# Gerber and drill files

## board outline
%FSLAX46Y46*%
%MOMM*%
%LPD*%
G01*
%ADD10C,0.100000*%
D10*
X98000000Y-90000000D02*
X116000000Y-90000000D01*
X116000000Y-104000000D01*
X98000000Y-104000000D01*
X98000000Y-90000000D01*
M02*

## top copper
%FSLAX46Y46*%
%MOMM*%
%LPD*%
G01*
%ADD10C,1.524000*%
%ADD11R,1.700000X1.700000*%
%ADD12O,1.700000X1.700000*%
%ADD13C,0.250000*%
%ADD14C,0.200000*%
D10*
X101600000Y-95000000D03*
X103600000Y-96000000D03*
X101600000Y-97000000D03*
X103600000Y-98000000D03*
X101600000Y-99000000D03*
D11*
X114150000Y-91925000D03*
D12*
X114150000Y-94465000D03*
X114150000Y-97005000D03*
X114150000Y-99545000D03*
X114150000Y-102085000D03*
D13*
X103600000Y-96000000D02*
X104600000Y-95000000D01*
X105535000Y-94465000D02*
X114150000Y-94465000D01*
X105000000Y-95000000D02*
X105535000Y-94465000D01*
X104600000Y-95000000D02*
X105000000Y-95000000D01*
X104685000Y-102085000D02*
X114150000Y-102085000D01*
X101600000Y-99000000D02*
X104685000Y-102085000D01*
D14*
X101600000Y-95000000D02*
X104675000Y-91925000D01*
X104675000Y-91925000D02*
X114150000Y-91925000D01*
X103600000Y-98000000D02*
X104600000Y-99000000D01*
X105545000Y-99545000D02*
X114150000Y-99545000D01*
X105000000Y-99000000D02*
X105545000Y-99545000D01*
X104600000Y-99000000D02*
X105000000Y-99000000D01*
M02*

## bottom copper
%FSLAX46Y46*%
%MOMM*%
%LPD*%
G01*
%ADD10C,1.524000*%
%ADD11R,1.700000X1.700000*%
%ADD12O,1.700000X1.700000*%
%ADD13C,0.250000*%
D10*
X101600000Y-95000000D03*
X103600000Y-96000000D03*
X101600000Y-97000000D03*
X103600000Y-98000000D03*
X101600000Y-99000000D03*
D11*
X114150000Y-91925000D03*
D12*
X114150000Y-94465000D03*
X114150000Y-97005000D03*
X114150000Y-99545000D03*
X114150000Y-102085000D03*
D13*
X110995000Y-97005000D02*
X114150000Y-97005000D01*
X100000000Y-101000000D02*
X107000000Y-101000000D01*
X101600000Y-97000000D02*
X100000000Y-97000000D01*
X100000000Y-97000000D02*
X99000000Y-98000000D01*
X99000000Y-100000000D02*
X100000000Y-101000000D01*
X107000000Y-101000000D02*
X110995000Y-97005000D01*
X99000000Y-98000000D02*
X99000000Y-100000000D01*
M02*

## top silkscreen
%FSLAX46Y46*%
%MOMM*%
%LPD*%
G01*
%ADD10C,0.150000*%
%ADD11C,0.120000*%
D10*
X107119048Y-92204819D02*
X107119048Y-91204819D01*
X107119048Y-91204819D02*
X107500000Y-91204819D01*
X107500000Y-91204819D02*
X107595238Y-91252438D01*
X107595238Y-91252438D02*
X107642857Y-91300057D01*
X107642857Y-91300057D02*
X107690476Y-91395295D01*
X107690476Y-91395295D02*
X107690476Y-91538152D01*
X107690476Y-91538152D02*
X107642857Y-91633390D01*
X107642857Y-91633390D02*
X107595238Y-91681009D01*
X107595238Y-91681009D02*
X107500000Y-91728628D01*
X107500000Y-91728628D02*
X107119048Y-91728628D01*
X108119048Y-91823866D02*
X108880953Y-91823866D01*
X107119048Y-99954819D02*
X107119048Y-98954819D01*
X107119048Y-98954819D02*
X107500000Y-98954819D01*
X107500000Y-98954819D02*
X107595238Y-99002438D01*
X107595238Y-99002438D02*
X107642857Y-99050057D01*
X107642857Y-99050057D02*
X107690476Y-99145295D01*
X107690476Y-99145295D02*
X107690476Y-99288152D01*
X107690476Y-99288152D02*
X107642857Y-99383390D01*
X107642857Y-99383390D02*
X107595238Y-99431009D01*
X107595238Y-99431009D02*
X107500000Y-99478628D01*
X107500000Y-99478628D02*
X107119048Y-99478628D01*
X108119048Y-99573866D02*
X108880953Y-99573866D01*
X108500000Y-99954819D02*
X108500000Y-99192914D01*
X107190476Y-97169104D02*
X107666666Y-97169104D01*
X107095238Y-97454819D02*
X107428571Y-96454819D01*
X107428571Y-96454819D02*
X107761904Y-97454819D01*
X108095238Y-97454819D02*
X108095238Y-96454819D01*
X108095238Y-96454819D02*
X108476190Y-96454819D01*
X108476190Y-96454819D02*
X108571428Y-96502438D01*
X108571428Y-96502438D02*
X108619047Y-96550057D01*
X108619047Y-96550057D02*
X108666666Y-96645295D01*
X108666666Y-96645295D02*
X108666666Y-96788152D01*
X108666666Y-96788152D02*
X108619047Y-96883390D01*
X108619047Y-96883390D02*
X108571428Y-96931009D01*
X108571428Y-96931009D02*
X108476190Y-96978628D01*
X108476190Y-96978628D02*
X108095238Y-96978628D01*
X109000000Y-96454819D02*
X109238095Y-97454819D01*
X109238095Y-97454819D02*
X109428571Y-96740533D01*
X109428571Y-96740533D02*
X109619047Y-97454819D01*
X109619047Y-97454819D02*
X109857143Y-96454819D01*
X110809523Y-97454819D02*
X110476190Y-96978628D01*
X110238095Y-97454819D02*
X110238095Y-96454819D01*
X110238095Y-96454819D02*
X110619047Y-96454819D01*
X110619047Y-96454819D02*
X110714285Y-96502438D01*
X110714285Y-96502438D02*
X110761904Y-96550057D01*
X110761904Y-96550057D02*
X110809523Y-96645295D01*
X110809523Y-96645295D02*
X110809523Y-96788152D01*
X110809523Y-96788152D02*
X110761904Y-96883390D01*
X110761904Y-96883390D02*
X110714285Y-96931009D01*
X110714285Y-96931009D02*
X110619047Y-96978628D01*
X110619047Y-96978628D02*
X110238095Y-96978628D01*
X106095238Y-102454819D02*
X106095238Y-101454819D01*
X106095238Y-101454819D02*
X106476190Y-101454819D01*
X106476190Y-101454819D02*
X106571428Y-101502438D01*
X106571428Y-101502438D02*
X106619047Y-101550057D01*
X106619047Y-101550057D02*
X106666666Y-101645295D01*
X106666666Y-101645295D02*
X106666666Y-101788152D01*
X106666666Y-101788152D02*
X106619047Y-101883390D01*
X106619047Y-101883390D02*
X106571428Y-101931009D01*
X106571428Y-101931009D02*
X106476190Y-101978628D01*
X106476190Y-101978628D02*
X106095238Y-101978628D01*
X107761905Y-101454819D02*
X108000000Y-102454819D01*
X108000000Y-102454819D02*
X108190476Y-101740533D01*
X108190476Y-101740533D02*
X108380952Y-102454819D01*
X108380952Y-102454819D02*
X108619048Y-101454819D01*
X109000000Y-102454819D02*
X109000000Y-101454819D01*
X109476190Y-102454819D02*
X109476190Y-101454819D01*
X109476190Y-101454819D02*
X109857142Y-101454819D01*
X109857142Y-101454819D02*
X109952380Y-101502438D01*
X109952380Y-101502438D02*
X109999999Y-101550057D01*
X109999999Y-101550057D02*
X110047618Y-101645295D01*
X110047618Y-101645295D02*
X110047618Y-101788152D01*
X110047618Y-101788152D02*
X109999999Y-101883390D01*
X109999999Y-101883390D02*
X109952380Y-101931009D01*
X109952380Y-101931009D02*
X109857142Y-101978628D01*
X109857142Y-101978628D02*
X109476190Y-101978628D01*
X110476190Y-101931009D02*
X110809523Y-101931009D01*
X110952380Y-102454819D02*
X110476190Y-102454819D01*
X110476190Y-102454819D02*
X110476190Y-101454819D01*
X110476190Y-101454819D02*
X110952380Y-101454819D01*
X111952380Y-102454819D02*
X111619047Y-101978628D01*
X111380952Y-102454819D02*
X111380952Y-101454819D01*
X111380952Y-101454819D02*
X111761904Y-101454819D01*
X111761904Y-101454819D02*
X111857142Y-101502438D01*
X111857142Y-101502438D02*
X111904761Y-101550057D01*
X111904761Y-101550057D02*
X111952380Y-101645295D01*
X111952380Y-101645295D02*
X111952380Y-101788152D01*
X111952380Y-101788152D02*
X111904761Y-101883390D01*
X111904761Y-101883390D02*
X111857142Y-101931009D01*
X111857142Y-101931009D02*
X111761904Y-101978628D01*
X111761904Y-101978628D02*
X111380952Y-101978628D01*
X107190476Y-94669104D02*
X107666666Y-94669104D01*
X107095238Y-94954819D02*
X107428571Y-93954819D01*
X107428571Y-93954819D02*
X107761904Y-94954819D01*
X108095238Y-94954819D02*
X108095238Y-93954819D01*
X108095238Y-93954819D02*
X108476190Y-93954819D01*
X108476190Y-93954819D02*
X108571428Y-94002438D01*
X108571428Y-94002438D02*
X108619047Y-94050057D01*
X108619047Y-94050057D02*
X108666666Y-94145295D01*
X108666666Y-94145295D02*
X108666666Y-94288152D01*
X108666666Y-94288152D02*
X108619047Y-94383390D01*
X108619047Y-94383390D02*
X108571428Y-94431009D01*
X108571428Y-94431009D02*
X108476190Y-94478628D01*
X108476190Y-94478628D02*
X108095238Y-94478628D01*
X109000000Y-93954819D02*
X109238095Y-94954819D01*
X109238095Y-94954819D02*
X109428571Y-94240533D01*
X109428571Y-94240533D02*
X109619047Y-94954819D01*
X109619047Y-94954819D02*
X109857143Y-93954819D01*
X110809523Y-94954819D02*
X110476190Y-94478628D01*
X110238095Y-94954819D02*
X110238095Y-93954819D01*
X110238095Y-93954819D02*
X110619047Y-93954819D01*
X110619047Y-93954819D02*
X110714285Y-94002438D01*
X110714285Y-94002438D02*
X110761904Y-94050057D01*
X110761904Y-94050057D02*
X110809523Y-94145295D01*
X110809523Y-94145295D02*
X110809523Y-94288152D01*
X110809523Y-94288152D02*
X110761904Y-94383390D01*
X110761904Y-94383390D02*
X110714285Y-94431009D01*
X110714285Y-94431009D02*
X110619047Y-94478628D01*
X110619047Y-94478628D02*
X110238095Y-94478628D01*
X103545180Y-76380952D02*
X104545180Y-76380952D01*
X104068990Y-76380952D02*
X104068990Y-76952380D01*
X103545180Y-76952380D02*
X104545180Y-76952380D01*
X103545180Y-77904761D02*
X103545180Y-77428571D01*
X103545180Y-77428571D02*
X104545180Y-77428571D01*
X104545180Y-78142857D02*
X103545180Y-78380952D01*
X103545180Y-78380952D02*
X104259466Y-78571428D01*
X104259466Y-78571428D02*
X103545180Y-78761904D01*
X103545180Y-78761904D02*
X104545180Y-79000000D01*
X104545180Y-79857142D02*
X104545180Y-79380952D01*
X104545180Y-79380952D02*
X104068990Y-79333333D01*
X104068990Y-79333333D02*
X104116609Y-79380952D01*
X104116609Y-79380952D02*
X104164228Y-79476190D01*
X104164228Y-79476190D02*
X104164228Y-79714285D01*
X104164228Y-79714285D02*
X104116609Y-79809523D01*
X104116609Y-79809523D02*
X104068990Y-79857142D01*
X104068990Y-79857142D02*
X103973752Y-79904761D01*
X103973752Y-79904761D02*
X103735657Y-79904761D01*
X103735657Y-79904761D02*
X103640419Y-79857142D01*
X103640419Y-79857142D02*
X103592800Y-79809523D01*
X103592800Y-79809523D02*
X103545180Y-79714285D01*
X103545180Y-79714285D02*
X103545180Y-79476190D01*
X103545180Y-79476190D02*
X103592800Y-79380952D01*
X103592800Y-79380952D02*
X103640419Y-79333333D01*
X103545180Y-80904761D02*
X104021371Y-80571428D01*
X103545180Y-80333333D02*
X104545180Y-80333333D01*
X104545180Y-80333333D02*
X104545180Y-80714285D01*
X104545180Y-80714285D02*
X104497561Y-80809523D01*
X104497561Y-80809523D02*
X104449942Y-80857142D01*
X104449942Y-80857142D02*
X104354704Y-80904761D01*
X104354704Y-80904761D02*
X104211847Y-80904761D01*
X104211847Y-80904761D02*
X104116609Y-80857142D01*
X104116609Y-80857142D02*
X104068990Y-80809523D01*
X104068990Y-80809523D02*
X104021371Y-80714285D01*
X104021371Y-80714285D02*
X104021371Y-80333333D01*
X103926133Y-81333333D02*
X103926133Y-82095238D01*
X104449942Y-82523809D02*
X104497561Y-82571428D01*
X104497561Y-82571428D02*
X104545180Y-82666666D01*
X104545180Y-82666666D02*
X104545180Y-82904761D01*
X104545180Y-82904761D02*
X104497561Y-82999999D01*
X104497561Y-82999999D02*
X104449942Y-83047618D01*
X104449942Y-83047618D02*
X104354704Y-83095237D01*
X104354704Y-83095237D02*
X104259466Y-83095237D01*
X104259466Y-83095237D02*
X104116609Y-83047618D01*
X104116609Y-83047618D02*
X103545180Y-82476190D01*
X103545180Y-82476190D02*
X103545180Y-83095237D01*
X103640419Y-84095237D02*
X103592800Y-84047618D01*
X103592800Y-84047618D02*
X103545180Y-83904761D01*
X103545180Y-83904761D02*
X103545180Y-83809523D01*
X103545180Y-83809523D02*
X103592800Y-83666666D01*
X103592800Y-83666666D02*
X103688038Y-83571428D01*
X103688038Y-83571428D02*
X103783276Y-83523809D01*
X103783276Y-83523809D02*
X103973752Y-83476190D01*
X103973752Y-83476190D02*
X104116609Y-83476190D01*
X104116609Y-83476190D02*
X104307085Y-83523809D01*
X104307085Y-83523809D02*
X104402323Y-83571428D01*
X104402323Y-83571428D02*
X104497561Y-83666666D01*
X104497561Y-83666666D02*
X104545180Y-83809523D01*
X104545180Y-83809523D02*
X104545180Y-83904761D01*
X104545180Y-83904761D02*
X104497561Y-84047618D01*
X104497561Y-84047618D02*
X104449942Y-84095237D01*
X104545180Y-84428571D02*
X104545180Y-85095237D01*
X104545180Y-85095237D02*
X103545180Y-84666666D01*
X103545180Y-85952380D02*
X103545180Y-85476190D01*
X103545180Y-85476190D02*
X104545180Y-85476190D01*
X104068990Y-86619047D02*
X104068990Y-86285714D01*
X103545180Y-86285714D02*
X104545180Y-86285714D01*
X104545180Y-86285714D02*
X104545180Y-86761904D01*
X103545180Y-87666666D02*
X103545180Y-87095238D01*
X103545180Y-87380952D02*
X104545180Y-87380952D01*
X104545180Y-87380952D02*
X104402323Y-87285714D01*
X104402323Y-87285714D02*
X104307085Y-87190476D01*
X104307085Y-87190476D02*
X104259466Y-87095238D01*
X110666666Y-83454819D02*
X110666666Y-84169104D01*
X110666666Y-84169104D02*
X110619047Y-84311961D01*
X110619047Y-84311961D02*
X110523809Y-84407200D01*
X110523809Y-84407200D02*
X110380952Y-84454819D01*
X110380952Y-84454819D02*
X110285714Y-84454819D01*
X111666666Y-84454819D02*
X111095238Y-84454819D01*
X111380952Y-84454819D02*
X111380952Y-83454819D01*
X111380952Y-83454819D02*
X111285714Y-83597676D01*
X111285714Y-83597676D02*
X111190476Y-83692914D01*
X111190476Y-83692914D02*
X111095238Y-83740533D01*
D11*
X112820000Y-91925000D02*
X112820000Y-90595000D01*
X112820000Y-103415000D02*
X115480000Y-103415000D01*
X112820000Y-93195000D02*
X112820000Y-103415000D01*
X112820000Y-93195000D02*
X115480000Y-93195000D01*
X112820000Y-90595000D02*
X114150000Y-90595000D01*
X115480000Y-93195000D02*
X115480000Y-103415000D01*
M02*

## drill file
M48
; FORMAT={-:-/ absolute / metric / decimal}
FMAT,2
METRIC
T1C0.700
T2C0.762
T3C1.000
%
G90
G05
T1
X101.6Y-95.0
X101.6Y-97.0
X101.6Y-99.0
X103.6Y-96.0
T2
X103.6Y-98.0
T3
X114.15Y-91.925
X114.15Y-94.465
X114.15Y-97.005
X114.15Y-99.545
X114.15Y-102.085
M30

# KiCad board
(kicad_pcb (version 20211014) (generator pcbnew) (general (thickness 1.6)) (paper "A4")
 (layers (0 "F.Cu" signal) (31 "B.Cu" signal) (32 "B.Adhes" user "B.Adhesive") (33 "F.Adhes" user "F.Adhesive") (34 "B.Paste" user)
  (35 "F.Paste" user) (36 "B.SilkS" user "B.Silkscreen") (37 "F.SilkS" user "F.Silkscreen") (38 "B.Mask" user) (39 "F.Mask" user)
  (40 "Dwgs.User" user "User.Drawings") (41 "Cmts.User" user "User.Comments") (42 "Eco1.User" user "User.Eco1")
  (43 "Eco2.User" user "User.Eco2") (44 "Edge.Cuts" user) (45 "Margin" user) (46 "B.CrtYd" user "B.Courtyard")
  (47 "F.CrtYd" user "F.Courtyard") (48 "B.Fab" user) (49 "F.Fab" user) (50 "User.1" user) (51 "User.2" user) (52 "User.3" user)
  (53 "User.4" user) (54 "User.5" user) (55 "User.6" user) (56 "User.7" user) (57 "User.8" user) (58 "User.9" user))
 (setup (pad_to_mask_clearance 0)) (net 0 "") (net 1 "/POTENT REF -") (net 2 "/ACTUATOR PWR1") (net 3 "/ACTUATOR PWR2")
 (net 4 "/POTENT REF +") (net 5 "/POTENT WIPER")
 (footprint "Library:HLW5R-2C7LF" (layer "F.Cu") (at 101.6 95 -90)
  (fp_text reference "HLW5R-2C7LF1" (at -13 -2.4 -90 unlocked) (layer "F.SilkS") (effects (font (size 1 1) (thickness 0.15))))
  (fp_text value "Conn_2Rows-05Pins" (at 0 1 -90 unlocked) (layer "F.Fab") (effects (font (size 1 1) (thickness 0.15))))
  (pad "1" thru_hole circle (at 0 0 270) (size 1.524 1.524) (drill 0.7) (layers *.Cu *.Mask) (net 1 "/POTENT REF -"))
  (pad "2" thru_hole circle (at 1 -2 270) (size 1.524 1.524) (drill 0.7) (layers *.Cu *.Mask) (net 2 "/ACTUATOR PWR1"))
  (pad "3" thru_hole circle (at 2 0 270) (size 1.524 1.524) (drill 0.7) (layers *.Cu *.Mask) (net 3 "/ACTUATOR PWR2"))
  (pad "4" thru_hole circle (at 3 -2 270) (size 1.524 1.524) (drill 0.762) (layers *.Cu *.Mask) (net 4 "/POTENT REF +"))
  (pad "5" thru_hole circle (at 4 0 270) (size 1.524 1.524) (drill 0.7) (layers *.Cu *.Mask) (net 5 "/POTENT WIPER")))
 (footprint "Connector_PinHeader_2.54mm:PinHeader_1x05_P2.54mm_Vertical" (layer "F.Cu") (at 114.15 91.925)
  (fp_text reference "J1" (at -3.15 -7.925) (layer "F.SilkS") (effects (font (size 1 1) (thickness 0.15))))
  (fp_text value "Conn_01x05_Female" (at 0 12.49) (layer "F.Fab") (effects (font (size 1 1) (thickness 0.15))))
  (fp_line (start -1.33 0) (end -1.33 -1.33) (layer "F.SilkS") (width 0.12))
  (fp_line (start -1.33 11.49) (end 1.33 11.49) (layer "F.SilkS") (width 0.12))
  (fp_line (start -1.33 1.27) (end -1.33 11.49) (layer "F.SilkS") (width 0.12))
  (fp_line (start -1.33 1.27) (end 1.33 1.27) (layer "F.SilkS") (width 0.12))
  (fp_line (start -1.33 -1.33) (end 0 -1.33) (layer "F.SilkS") (width 0.12))
  (fp_line (start 1.33 1.27) (end 1.33 11.49) (layer "F.SilkS") (width 0.12))
  (pad "1" thru_hole rect locked (at 0 0) (size 1.7 1.7) (drill 1) (layers *.Cu *.Mask) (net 1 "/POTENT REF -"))
  (pad "2" thru_hole oval locked (at 0 2.54) (size 1.7 1.7) (drill 1) (layers *.Cu *.Mask) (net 2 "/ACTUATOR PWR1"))
  (pad "3" thru_hole oval locked (at 0 5.08) (size 1.7 1.7) (drill 1) (layers *.Cu *.Mask) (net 3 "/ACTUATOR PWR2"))
  (pad "4" thru_hole oval locked (at 0 7.62) (size 1.7 1.7) (drill 1) (layers *.Cu *.Mask) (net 4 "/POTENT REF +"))
  (pad "5" thru_hole oval locked (at 0 10.16) (size 1.7 1.7) (drill 1) (layers *.Cu *.Mask) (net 5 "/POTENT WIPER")))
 (gr_rect (start 116 90) (end 98 104) (layer "Edge.Cuts") (width 0.1) (fill none))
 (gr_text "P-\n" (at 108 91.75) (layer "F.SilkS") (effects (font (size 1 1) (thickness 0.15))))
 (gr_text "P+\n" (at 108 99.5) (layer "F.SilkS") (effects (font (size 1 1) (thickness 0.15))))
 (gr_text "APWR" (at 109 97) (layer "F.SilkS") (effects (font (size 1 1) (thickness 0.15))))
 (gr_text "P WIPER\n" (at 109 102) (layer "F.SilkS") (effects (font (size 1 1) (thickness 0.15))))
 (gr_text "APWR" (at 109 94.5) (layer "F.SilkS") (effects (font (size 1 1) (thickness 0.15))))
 (segment (start 103.6 96) (end 104.6 95) (width 0.25) (layer "F.Cu") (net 2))
 (segment (start 105.535 94.465) (end 114.15 94.465) (width 0.25) (layer "F.Cu") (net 2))
 (segment (start 105 95) (end 105.535 94.465) (width 0.25) (layer "F.Cu") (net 2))
 (segment (start 104.6 95) (end 105 95) (width 0.25) (layer "F.Cu") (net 2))
 (segment (start 110.995 97.005) (end 114.15 97.005) (width 0.25) (layer "B.Cu") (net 3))
 (segment (start 100 101) (end 107 101) (width 0.25) (layer "B.Cu") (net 3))
 (segment (start 101.6 97) (end 100 97) (width 0.25) (layer "B.Cu") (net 3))
 (segment (start 100 97) (end 99 98) (width 0.25) (layer "B.Cu") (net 3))
 (segment (start 99 100) (end 100 101) (width 0.25) (layer "B.Cu") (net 3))
 (segment (start 107 101) (end 110.995 97.005) (width 0.25) (layer "B.Cu") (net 3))
 (segment (start 99 98) (end 99 100) (width 0.25) (layer "B.Cu") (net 3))
 (segment (start 104.685 102.085) (end 114.15 102.085) (width 0.25) (layer "F.Cu") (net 5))
 (segment (start 101.6 99) (end 104.685 102.085) (width 0.25) (layer "F.Cu") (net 5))
 (segment (start 101.6 95) (end 104.675 91.925) (width 0.2) (layer "F.Cu") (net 1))
 (segment (start 104.675 91.925) (end 114.15 91.925) (width 0.2) (layer "F.Cu") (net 1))
 (segment (start 103.6 98) (end 104.6 99) (width 0.2) (layer "F.Cu") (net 4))
 (segment (start 105.545 99.545) (end 114.15 99.545) (width 0.2) (layer "F.Cu") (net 4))
 (segment (start 105 99) (end 105.545 99.545) (width 0.2) (layer "F.Cu") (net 4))
 (segment (start 104.6 99) (end 105 99) (width 0.2) (layer "F.Cu") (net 4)))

